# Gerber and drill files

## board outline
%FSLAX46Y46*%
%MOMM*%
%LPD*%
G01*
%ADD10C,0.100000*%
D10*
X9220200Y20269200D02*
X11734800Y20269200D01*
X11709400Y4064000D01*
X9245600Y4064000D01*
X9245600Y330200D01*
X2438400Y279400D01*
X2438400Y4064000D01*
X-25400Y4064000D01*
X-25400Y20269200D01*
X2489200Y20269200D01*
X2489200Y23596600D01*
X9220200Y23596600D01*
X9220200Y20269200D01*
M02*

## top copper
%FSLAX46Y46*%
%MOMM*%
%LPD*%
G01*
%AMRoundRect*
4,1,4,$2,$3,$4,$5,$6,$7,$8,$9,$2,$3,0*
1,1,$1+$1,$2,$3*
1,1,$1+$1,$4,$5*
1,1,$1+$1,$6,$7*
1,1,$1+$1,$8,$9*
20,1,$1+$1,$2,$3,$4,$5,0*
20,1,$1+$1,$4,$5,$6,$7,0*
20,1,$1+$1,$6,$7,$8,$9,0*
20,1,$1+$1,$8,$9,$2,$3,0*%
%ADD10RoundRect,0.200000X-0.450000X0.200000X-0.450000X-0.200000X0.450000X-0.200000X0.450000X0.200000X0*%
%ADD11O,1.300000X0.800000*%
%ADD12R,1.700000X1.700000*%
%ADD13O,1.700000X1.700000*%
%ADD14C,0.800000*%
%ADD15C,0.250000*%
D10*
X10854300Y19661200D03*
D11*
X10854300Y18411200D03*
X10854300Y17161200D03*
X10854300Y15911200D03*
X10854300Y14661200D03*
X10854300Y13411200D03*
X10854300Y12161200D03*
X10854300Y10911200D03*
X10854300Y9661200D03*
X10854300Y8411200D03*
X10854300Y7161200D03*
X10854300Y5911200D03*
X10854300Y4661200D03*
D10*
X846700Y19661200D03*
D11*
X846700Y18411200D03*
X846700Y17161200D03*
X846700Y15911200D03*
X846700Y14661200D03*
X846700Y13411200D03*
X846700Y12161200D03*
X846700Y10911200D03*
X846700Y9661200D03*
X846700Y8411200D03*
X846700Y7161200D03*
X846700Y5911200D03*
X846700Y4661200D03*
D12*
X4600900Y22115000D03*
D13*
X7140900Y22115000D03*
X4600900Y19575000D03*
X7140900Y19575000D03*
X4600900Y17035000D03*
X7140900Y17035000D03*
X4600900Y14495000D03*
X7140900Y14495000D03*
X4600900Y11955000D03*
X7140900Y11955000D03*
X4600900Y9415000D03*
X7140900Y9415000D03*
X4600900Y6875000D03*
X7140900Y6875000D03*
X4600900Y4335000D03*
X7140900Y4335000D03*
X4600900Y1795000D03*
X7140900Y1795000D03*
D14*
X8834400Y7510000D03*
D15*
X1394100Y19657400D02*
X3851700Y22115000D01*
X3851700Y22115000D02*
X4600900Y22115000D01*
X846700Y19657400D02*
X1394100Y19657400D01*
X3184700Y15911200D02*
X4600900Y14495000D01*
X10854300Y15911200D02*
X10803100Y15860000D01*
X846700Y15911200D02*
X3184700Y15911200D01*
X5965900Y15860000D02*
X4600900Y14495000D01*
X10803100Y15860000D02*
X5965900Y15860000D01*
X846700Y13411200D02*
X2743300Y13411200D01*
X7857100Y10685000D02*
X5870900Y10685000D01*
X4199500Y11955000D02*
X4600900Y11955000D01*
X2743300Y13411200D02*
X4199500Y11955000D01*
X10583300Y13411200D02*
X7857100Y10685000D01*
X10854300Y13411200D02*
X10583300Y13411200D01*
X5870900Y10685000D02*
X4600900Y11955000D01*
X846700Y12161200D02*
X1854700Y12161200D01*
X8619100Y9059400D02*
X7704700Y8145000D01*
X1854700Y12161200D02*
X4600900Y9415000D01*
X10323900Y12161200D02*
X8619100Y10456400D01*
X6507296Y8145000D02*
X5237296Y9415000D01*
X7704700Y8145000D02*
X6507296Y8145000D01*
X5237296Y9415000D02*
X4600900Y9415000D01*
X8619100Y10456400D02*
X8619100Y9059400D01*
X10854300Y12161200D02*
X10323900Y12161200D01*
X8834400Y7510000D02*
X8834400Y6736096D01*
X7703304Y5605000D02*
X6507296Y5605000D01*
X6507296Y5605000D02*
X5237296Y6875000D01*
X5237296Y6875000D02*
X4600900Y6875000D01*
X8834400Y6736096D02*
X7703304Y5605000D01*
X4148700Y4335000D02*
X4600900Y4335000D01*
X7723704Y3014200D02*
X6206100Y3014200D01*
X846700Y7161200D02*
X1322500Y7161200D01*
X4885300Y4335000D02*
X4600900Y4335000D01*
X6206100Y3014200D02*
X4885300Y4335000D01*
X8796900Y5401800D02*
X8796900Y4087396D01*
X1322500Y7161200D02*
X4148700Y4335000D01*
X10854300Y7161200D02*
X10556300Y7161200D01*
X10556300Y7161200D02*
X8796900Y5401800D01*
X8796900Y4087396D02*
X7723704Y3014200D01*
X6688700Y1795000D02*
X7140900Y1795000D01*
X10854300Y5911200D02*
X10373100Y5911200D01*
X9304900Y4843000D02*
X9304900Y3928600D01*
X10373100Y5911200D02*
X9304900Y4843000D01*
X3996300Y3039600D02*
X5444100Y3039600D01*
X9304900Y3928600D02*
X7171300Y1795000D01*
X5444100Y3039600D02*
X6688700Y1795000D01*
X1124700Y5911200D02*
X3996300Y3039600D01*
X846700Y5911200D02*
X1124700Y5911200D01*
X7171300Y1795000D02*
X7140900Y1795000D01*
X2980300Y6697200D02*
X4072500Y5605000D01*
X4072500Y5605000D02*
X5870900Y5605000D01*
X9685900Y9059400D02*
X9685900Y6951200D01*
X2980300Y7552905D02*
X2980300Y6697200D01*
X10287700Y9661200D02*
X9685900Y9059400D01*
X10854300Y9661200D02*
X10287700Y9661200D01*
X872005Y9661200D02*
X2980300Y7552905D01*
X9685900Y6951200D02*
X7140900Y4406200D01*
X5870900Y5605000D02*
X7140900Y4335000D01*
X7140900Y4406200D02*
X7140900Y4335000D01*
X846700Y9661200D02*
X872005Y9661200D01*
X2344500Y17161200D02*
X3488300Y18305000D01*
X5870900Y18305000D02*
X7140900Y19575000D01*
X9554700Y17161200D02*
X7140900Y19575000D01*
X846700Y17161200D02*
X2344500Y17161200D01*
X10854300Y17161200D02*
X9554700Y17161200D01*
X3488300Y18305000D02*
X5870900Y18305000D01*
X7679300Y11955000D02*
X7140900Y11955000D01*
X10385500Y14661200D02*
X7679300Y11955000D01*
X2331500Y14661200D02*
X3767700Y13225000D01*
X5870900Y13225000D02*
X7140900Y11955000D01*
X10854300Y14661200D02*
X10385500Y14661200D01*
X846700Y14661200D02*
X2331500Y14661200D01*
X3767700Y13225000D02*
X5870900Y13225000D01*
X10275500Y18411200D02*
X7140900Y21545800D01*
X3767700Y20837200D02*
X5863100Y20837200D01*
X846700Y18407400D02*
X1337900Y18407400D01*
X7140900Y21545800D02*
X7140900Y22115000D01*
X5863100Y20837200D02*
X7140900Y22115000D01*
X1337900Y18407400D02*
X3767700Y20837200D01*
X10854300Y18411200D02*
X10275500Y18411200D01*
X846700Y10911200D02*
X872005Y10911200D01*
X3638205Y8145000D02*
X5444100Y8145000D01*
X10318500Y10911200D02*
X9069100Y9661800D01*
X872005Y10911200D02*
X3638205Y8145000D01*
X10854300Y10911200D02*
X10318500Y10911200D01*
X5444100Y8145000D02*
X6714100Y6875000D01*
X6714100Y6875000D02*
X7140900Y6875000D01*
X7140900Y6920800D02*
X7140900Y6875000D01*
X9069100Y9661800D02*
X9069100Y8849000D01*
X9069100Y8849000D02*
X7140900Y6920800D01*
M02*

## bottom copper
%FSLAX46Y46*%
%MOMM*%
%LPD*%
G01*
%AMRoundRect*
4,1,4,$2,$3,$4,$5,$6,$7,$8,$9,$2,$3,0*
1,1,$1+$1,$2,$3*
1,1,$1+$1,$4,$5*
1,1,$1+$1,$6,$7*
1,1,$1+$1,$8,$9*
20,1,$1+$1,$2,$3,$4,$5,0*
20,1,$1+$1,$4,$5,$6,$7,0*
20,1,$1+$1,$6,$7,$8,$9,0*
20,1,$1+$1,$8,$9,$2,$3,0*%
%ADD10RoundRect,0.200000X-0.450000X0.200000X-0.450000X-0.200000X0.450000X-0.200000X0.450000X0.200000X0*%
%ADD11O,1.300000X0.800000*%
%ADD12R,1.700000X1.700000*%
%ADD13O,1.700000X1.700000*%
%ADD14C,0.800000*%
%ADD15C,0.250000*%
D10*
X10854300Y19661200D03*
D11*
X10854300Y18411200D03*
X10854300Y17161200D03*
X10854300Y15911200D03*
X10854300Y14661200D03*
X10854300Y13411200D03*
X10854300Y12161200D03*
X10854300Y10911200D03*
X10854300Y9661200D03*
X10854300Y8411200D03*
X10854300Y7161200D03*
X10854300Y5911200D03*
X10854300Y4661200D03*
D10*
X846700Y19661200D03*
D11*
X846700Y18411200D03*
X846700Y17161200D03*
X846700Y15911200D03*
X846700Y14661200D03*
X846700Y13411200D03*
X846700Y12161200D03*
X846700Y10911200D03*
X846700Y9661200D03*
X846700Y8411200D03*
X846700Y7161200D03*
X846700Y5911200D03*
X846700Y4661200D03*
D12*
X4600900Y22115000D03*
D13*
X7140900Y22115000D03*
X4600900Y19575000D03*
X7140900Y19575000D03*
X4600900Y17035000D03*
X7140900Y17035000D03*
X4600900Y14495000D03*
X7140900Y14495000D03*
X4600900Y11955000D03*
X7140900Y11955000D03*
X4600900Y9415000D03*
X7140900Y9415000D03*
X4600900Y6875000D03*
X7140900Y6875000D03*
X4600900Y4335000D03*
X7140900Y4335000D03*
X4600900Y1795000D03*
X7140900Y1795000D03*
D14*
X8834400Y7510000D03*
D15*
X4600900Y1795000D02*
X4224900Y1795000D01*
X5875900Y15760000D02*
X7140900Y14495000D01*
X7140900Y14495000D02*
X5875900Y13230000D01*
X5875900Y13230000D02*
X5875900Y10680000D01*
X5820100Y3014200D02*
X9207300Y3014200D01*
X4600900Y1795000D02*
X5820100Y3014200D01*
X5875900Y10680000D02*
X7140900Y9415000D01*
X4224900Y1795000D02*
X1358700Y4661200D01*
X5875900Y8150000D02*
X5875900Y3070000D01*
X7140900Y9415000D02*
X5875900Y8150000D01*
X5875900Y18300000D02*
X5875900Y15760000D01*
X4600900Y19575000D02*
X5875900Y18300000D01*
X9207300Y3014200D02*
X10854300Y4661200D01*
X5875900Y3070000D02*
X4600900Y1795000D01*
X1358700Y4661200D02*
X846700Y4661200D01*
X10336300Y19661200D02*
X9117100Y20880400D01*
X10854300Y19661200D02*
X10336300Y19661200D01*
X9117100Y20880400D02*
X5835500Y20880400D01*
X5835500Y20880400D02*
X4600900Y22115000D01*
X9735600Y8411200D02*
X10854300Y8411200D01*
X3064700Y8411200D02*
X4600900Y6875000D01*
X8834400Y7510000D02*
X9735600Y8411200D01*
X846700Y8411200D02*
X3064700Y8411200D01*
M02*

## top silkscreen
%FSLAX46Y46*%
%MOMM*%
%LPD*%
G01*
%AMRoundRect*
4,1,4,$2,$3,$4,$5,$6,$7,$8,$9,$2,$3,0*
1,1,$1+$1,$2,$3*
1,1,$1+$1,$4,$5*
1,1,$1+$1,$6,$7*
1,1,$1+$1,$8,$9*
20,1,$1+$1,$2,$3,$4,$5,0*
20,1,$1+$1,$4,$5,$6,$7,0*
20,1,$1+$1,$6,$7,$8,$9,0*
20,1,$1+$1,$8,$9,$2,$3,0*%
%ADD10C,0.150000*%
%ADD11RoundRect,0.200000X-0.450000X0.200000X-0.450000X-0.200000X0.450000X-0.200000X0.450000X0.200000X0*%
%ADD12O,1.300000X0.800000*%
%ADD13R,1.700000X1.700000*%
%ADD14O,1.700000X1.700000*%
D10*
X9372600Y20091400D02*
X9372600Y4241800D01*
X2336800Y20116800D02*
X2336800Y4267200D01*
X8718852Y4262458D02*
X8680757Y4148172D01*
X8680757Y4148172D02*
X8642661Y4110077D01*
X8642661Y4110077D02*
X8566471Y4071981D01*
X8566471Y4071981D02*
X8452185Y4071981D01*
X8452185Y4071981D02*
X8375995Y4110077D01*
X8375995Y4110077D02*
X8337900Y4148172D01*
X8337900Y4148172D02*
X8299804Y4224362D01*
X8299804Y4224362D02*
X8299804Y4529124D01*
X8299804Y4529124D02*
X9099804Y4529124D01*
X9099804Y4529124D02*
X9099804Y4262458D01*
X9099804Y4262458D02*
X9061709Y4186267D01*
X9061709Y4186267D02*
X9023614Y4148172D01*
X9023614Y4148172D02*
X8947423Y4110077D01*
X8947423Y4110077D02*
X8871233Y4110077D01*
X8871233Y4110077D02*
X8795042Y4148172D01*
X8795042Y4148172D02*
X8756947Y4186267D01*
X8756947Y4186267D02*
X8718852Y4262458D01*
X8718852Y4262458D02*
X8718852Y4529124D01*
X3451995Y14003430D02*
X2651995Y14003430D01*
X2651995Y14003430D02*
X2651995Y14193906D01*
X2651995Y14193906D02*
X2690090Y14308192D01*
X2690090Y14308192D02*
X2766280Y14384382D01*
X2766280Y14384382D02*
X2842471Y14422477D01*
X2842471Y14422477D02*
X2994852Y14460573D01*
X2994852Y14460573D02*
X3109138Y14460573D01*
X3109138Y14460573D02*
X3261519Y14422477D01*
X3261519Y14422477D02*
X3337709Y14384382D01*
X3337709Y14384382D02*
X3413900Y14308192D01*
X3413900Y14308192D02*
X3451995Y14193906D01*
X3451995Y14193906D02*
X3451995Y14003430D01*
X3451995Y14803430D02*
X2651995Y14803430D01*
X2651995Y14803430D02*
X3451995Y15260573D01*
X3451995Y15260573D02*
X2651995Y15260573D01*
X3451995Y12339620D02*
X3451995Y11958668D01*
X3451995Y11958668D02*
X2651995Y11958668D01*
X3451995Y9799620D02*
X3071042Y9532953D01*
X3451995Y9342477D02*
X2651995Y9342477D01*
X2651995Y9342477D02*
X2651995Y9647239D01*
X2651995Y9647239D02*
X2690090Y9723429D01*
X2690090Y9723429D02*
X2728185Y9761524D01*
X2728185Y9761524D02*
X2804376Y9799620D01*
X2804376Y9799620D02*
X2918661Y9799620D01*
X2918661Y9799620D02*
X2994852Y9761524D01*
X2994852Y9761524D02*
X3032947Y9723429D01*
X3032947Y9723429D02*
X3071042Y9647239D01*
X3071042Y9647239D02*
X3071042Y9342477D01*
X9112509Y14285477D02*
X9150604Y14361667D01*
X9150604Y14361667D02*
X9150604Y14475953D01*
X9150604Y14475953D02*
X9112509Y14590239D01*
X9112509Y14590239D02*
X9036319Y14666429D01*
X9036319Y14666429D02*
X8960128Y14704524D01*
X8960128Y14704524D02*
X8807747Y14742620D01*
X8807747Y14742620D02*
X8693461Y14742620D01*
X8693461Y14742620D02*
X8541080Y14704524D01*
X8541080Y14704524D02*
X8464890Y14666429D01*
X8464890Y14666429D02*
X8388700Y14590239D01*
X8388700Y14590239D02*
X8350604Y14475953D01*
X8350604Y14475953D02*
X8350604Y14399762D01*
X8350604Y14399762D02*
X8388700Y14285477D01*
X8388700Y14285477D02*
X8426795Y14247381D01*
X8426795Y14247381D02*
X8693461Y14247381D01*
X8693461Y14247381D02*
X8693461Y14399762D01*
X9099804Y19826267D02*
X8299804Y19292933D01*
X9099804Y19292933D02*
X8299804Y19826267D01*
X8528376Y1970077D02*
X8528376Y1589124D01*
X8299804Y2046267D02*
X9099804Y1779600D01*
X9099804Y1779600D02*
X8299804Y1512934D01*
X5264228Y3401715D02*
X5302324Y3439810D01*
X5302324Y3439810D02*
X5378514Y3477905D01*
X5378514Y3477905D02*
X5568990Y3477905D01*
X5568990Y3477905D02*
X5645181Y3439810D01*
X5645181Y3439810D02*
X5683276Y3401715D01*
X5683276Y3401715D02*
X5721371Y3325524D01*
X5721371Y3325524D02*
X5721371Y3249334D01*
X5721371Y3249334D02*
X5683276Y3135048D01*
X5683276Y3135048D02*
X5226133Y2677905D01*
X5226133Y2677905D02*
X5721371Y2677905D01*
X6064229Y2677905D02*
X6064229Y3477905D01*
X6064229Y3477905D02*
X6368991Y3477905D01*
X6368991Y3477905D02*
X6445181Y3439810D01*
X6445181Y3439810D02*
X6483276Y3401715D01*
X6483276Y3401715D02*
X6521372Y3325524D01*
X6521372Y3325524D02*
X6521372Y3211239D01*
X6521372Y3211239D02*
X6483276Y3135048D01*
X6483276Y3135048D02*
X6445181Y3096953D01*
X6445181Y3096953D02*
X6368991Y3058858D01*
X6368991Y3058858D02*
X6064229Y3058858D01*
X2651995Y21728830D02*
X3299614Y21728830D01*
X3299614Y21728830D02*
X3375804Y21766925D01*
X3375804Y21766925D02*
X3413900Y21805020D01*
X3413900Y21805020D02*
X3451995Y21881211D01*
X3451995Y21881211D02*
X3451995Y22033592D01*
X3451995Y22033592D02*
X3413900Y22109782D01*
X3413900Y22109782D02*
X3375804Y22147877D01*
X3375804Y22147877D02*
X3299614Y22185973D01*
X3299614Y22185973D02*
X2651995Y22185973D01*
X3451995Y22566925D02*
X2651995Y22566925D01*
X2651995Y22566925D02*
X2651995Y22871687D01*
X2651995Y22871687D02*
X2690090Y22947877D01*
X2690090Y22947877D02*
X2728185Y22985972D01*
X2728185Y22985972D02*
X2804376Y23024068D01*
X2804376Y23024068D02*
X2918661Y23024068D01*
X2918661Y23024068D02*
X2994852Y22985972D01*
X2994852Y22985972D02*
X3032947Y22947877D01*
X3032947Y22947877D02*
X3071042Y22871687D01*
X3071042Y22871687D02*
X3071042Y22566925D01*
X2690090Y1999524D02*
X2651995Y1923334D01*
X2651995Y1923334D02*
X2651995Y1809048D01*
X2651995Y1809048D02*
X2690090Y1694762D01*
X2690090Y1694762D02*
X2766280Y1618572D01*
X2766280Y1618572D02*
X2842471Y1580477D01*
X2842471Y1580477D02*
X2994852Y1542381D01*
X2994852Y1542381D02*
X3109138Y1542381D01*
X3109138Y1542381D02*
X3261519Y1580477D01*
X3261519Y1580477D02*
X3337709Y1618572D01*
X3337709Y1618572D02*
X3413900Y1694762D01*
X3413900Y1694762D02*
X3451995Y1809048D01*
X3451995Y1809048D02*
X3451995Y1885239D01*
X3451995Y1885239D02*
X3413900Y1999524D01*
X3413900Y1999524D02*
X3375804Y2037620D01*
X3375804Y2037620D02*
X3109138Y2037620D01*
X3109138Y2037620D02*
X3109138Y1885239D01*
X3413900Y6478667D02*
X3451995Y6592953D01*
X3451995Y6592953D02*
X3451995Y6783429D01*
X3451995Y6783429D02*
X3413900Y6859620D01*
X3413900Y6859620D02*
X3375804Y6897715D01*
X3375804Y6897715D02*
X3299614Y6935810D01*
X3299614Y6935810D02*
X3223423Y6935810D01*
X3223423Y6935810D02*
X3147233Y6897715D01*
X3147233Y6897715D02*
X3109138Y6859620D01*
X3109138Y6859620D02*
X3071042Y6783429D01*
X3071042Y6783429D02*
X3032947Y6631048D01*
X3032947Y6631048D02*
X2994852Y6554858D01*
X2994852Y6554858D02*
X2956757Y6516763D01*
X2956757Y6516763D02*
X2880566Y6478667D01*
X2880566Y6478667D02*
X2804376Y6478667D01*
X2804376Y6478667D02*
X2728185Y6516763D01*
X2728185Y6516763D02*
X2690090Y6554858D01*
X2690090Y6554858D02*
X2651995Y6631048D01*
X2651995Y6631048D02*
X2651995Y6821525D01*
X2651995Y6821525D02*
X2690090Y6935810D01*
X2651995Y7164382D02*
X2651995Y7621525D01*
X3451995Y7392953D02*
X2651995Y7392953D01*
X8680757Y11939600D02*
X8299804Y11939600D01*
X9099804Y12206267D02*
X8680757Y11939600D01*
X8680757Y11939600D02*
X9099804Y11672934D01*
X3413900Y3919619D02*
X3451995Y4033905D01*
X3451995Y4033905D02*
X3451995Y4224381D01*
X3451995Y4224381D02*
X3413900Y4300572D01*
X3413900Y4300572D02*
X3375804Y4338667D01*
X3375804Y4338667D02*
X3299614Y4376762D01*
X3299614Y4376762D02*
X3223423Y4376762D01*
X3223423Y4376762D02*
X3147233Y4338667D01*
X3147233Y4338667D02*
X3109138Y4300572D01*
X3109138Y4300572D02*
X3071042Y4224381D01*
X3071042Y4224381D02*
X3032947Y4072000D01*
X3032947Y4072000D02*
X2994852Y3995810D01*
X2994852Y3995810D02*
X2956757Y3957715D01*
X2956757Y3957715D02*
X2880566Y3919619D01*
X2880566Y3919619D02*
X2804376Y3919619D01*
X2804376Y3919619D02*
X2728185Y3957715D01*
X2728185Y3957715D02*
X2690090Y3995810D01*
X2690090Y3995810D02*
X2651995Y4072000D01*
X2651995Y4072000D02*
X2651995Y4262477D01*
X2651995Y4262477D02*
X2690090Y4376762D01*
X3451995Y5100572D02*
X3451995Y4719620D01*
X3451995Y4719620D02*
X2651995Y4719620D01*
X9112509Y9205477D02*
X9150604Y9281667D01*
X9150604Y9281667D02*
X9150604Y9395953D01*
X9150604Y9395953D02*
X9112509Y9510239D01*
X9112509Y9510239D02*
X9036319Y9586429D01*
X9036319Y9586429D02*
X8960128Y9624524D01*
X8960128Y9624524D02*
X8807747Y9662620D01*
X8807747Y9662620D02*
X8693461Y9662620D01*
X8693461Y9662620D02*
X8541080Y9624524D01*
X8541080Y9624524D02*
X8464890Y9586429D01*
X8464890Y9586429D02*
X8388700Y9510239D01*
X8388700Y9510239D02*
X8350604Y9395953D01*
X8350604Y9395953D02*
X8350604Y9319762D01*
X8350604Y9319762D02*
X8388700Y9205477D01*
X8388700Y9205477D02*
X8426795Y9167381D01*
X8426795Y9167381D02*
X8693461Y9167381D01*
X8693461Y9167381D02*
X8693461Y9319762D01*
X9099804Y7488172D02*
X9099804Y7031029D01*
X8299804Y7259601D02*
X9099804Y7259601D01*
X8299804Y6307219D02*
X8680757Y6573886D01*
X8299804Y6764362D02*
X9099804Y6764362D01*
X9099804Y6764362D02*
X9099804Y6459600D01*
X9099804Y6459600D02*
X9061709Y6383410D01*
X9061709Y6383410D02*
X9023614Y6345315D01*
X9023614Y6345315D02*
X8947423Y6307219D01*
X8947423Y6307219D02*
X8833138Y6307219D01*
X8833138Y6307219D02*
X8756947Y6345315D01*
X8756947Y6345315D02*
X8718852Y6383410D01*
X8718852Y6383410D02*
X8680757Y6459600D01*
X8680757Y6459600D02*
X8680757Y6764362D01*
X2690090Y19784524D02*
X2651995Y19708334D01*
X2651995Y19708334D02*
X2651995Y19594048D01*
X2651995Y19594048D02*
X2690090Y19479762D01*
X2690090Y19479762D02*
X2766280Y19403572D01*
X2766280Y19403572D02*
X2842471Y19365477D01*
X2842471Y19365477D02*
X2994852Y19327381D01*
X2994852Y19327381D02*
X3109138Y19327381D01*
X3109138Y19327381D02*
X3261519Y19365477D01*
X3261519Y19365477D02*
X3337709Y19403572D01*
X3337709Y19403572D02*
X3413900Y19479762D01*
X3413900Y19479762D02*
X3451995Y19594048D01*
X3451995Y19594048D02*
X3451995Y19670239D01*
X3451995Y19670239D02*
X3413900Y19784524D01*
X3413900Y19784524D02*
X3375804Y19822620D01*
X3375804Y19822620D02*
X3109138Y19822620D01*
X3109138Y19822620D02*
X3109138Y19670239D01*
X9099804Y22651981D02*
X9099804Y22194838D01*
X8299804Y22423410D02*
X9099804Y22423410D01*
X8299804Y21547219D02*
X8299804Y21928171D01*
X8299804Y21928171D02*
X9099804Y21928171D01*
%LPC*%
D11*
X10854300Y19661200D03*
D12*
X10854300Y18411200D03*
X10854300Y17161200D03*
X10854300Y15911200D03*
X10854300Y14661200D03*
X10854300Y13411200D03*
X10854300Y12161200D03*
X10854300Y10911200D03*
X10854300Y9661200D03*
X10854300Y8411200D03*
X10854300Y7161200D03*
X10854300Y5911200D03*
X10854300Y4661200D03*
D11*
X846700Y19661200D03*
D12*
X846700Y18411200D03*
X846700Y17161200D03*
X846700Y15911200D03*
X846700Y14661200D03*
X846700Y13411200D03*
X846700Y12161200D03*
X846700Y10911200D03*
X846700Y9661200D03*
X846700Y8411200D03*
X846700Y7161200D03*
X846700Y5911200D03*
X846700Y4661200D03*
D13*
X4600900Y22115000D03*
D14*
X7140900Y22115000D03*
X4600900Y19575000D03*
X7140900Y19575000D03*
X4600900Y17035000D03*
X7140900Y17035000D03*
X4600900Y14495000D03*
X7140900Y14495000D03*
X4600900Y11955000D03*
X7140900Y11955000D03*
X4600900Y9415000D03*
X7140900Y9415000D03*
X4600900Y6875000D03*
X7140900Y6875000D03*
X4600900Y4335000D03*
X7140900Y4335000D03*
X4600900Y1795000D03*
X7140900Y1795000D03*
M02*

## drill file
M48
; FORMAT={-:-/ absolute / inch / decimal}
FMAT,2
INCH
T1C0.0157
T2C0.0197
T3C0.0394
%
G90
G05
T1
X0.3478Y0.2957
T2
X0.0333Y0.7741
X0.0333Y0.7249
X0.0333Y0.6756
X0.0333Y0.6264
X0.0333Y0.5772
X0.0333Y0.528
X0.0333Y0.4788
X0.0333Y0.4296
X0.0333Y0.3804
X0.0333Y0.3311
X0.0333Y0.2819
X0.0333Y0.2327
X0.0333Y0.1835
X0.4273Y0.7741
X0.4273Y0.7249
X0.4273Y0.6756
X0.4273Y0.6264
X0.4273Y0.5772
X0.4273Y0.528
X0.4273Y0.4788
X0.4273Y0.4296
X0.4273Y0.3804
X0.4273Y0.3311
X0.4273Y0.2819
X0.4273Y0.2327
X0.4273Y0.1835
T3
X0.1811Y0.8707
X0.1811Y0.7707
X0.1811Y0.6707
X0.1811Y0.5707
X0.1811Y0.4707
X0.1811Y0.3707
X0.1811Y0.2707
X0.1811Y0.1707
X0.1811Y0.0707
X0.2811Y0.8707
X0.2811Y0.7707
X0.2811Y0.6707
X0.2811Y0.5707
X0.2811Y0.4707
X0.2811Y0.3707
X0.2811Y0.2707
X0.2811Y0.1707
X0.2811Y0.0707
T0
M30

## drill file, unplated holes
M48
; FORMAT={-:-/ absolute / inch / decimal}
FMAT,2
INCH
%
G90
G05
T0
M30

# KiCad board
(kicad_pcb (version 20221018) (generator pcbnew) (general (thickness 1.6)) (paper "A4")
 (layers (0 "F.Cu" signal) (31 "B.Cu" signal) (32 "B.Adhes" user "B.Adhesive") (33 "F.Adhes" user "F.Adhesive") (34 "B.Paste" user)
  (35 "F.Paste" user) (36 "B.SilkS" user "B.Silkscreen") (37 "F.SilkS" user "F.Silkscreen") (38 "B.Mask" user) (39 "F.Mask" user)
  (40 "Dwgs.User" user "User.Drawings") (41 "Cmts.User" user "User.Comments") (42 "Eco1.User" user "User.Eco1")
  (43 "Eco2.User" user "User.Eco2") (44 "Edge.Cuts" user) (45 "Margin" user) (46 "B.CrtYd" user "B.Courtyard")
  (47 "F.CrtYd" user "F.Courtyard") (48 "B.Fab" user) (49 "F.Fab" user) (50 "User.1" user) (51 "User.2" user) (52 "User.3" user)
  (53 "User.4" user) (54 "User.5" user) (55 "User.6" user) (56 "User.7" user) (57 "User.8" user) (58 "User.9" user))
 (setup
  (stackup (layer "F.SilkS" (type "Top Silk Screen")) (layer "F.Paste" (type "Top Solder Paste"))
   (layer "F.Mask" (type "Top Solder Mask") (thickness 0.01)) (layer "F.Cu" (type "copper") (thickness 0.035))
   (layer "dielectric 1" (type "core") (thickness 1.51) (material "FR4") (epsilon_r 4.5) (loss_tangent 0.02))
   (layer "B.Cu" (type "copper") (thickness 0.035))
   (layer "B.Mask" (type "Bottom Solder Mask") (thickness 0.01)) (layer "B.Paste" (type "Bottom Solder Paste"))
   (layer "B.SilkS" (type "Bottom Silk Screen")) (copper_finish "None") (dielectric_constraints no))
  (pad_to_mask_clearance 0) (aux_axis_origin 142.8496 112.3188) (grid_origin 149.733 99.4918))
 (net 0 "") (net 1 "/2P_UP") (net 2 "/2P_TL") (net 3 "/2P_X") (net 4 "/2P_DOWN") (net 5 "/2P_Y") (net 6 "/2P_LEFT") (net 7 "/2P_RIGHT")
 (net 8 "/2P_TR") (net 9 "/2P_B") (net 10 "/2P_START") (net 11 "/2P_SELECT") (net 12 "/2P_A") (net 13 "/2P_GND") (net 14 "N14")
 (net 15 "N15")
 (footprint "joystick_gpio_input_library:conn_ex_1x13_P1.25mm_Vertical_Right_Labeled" (layer "B.Cu") (at 153.7039 92.6576 -90)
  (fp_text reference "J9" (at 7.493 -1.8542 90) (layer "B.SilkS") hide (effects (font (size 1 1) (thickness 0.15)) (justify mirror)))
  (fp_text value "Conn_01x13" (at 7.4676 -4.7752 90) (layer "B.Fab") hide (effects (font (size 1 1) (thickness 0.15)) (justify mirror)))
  (pad "1" thru_hole roundrect (at 0 0 270) (size 0.8 1.3) (drill 0.5) (layers "*.Cu" "*.Mask") (roundrect_rratio 0.25) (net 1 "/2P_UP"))
  (pad "2" thru_hole oval (at 1.25 0 270) (size 0.8 1.3) (drill 0.5) (layers "*.Cu" "*.Mask") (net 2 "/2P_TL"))
  (pad "3" thru_hole oval (at 2.5 0 270) (size 0.8 1.3) (drill 0.5) (layers "*.Cu" "*.Mask") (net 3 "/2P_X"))
  (pad "4" thru_hole oval (at 3.75 0 270) (size 0.8 1.3) (drill 0.5) (layers "*.Cu" "*.Mask") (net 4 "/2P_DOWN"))
  (pad "5" thru_hole oval (at 5 0 270) (size 0.8 1.3) (drill 0.5) (layers "*.Cu" "*.Mask") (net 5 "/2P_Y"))
  (pad "6" thru_hole oval (at 6.25 0 270) (size 0.8 1.3) (drill 0.5) (layers "*.Cu" "*.Mask") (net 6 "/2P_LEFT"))
  (pad "7" thru_hole oval (at 7.5 0 270) (size 0.8 1.3) (drill 0.5) (layers "*.Cu" "*.Mask") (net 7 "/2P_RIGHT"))
  (pad "8" thru_hole oval (at 8.75 0 270) (size 0.8 1.3) (drill 0.5) (layers "*.Cu" "*.Mask") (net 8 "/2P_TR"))
  (pad "9" thru_hole oval (at 10 0 270) (size 0.8 1.3) (drill 0.5) (layers "*.Cu" "*.Mask") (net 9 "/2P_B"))
  (pad "10" thru_hole oval (at 11.25 0 270) (size 0.8 1.3) (drill 0.5) (layers "*.Cu" "*.Mask") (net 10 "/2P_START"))
  (pad "11" thru_hole oval (at 12.5 0 270) (size 0.8 1.3) (drill 0.5) (layers "*.Cu" "*.Mask") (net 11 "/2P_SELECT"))
  (pad "12" thru_hole oval (at 13.75 0 270) (size 0.8 1.3) (drill 0.5) (layers "*.Cu" "*.Mask") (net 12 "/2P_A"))
  (pad "13" thru_hole oval (at 15 0 270) (size 0.8 1.3) (drill 0.5) (layers "*.Cu" "*.Mask") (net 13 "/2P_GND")))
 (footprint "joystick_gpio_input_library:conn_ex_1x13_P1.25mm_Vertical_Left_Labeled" (layer "B.Cu") (at 143.6963 92.6576 -90)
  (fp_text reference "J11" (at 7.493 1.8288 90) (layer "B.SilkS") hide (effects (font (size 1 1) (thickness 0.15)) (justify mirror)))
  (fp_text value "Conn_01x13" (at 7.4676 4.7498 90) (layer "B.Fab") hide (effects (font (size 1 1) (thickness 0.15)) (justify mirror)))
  (pad "1" thru_hole roundrect (at 0 0 270) (size 0.8 1.3) (drill 0.5) (layers "*.Cu" "*.Mask") (roundrect_rratio 0.25) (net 1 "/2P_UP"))
  (pad "2" thru_hole oval (at 1.25 0 270) (size 0.8 1.3) (drill 0.5) (layers "*.Cu" "*.Mask") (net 2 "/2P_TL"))
  (pad "3" thru_hole oval (at 2.5 0 270) (size 0.8 1.3) (drill 0.5) (layers "*.Cu" "*.Mask") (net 3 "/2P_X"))
  (pad "4" thru_hole oval (at 3.75 0 270) (size 0.8 1.3) (drill 0.5) (layers "*.Cu" "*.Mask") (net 4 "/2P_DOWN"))
  (pad "5" thru_hole oval (at 5 0 270) (size 0.8 1.3) (drill 0.5) (layers "*.Cu" "*.Mask") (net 5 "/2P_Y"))
  (pad "6" thru_hole oval (at 6.25 0 270) (size 0.8 1.3) (drill 0.5) (layers "*.Cu" "*.Mask") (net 6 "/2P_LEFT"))
  (pad "7" thru_hole oval (at 7.5 0 270) (size 0.8 1.3) (drill 0.5) (layers "*.Cu" "*.Mask") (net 7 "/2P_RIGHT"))
  (pad "8" thru_hole oval (at 8.75 0 270) (size 0.8 1.3) (drill 0.5) (layers "*.Cu" "*.Mask") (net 8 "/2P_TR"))
  (pad "9" thru_hole oval (at 10 0 270) (size 0.8 1.3) (drill 0.5) (layers "*.Cu" "*.Mask") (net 9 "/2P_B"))
  (pad "10" thru_hole oval (at 11.25 0 270) (size 0.8 1.3) (drill 0.5) (layers "*.Cu" "*.Mask") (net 10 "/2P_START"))
  (pad "11" thru_hole oval (at 12.5 0 270) (size 0.8 1.3) (drill 0.5) (layers "*.Cu" "*.Mask") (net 11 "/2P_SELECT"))
  (pad "12" thru_hole oval (at 13.75 0 270) (size 0.8 1.3) (drill 0.5) (layers "*.Cu" "*.Mask") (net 12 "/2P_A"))
  (pad "13" thru_hole oval (at 15 0 270) (size 0.8 1.3) (drill 0.5) (layers "*.Cu" "*.Mask") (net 13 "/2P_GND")))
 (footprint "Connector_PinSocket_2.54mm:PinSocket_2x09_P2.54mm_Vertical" (layer "B.Cu") (at 147.4505 90.2038 180)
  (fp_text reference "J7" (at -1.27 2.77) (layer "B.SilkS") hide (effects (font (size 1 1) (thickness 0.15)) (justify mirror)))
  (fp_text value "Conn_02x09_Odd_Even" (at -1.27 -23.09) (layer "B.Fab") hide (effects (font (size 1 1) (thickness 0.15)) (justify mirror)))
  (pad "1" thru_hole rect (at 0 0 180) (size 1.7 1.7) (drill 1) (layers "*.Cu" "*.Mask") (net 1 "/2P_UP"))
  (pad "2" thru_hole oval (at -2.54 0 180) (size 1.7 1.7) (drill 1) (layers "*.Cu" "*.Mask") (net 2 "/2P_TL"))
  (pad "3" thru_hole oval (at 0 -2.54 180) (size 1.7 1.7) (drill 1) (layers "*.Cu" "*.Mask") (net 13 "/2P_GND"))
  (pad "4" thru_hole oval (at -2.54 -2.54 180) (size 1.7 1.7) (drill 1) (layers "*.Cu" "*.Mask") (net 3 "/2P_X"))
  (pad "5" thru_hole oval (at 0 -5.08 180) (size 1.7 1.7) (drill 1) (layers "*.Cu" "*.Mask") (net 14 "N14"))
  (pad "6" thru_hole oval (at -2.54 -5.08 180) (size 1.7 1.7) (drill 1) (layers "*.Cu" "*.Mask") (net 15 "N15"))
  (pad "7" thru_hole oval (at 0 -7.62 180) (size 1.7 1.7) (drill 1) (layers "*.Cu" "*.Mask") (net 4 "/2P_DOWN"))
  (pad "8" thru_hole oval (at -2.54 -7.62 180) (size 1.7 1.7) (drill 1) (layers "*.Cu" "*.Mask") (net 13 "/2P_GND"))
  (pad "9" thru_hole oval (at 0 -10.16 180) (size 1.7 1.7) (drill 1) (layers "*.Cu" "*.Mask") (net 6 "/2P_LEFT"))
  (pad "10" thru_hole oval (at -2.54 -10.16 180) (size 1.7 1.7) (drill 1) (layers "*.Cu" "*.Mask") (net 5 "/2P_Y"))
  (pad "11" thru_hole oval (at 0 -12.7 180) (size 1.7 1.7) (drill 1) (layers "*.Cu" "*.Mask") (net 7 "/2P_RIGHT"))
  (pad "12" thru_hole oval (at -2.54 -12.7 180) (size 1.7 1.7) (drill 1) (layers "*.Cu" "*.Mask") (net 13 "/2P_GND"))
  (pad "13" thru_hole oval (at 0 -15.24 180) (size 1.7 1.7) (drill 1) (layers "*.Cu" "*.Mask") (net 10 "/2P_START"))
  (pad "14" thru_hole oval (at -2.54 -15.24 180) (size 1.7 1.7) (drill 1) (layers "*.Cu" "*.Mask") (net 8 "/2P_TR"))
  (pad "15" thru_hole oval (at 0 -17.78 180) (size 1.7 1.7) (drill 1) (layers "*.Cu" "*.Mask") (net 11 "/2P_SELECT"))
  (pad "16" thru_hole oval (at -2.54 -17.78 180) (size 1.7 1.7) (drill 1) (layers "*.Cu" "*.Mask") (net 9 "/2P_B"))
  (pad "17" thru_hole oval (at 0 -20.32 180) (size 1.7 1.7) (drill 1) (layers "*.Cu" "*.Mask") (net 13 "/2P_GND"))
  (pad "18" thru_hole oval (at -2.54 -20.32 180) (size 1.7 1.7) (drill 1) (layers "*.Cu" "*.Mask") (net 12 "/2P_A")))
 (gr_line (start 152.2222 92.2274) (end 152.2222 108.077) (stroke (width 0.15) (type default)) (layer "F.SilkS"))
 (gr_line (start 145.1864 92.202) (end 145.1864 108.0516) (stroke (width 0.15) (type default)) (layer "F.SilkS"))
 (gr_poly
  (pts (xy 145.3388 92.0496) (xy 145.3388 88.7222) (xy 152.0698 88.7222) (xy 152.0698 92.0496) (xy 154.5844 92.0496) (xy 154.559 108.2548)
   (xy 152.0952 108.2548) (xy 152.0952 111.9886) (xy 145.288 112.0394) (xy 145.288 108.2548) (xy 142.8242 108.2548) (xy 142.8242 92.0496))
  (stroke (width 0.1) (type solid)) (fill none) (layer "Edge.Cuts"))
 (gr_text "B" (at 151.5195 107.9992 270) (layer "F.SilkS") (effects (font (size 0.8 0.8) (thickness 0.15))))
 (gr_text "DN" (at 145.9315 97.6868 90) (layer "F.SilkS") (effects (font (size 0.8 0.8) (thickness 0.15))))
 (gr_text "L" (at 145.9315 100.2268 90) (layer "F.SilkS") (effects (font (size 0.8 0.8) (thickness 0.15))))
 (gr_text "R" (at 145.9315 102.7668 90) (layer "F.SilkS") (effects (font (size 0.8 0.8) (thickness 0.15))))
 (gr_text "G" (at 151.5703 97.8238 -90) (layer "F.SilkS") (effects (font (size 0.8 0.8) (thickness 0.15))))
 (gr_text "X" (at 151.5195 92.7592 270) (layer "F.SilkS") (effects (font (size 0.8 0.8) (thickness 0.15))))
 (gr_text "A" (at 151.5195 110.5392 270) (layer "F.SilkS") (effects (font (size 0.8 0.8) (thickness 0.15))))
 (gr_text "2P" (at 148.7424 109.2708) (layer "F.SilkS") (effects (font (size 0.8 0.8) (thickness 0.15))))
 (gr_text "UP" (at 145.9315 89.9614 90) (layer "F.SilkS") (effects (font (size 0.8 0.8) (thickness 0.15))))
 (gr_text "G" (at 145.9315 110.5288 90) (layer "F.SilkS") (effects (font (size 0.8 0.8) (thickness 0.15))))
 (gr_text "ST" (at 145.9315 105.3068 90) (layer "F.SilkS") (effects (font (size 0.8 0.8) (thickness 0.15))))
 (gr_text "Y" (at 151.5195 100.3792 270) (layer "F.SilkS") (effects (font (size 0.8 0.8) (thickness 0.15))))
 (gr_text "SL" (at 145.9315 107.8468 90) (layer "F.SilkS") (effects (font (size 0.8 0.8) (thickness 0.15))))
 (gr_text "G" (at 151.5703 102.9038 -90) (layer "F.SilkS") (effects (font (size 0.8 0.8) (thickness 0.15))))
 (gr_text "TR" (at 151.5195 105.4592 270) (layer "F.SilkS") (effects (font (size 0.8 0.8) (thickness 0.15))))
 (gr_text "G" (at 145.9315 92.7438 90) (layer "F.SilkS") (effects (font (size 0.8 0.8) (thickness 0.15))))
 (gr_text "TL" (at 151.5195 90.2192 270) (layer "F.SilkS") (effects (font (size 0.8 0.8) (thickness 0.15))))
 (segment (start 147.4505 110.5238) (end 147.0745 110.5238) (width 0.25) (layer "B.Cu") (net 13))
 (segment (start 148.7255 96.5588) (end 149.9905 97.8238) (width 0.25) (layer "B.Cu") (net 13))
 (segment (start 149.9905 97.8238) (end 148.7255 99.0888) (width 0.25) (layer "B.Cu") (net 13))
 (segment (start 148.7255 99.0888) (end 148.7255 101.6388) (width 0.25) (layer "B.Cu") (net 13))
 (segment (start 148.6697 109.3046) (end 152.0569 109.3046) (width 0.25) (layer "B.Cu") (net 13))
 (segment (start 147.4505 110.5238) (end 148.6697 109.3046) (width 0.25) (layer "B.Cu") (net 13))
 (segment (start 148.7255 101.6388) (end 149.9905 102.9038) (width 0.25) (layer "B.Cu") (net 13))
 (segment (start 147.0745 110.5238) (end 144.2083 107.6576) (width 0.25) (layer "B.Cu") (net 13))
 (segment (start 148.7255 104.1688) (end 148.7255 109.2488) (width 0.25) (layer "B.Cu") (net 13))
 (segment (start 149.9905 102.9038) (end 148.7255 104.1688) (width 0.25) (layer "B.Cu") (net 13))
 (segment (start 148.7255 94.0188) (end 148.7255 96.5588) (width 0.25) (layer "B.Cu") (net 13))
 (segment (start 147.4505 92.7438) (end 148.7255 94.0188) (width 0.25) (layer "B.Cu") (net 13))
 (segment (start 152.0569 109.3046) (end 153.7039 107.6576) (width 0.25) (layer "B.Cu") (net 13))
 (segment (start 148.7255 109.2488) (end 147.4505 110.5238) (width 0.25) (layer "B.Cu") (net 13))
 (segment (start 144.2083 107.6576) (end 143.6963 107.6576) (width 0.25) (layer "B.Cu") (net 13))
 (segment (start 144.2437 92.6614) (end 146.7013 90.2038) (width 0.25) (layer "F.Cu") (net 1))
 (segment (start 146.7013 90.2038) (end 147.4505 90.2038) (width 0.25) (layer "F.Cu") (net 1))
 (segment (start 143.6963 92.6614) (end 144.2437 92.6614) (width 0.25) (layer "F.Cu") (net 1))
 (segment (start 153.1859 92.6576) (end 151.9667 91.4384) (width 0.25) (layer "B.Cu") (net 1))
 (segment (start 153.7039 92.6576) (end 153.1859 92.6576) (width 0.25) (layer "B.Cu") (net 1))
 (segment (start 151.9667 91.4384) (end 148.6851 91.4384) (width 0.25) (layer "B.Cu") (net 1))
 (segment (start 148.6851 91.4384) (end 147.4505 90.2038) (width 0.25) (layer "B.Cu") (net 1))
 (segment (start 146.0343 96.4076) (end 147.4505 97.8238) (width 0.25) (layer "F.Cu") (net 4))
 (segment (start 153.7039 96.4076) (end 153.6527 96.4588) (width 0.25) (layer "F.Cu") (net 4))
 (segment (start 143.6963 96.4076) (end 146.0343 96.4076) (width 0.25) (layer "F.Cu") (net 4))
 (segment (start 148.8155 96.4588) (end 147.4505 97.8238) (width 0.25) (layer "F.Cu") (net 4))
 (segment (start 153.6527 96.4588) (end 148.8155 96.4588) (width 0.25) (layer "F.Cu") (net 4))
 (segment (start 143.6963 98.9076) (end 145.5929 98.9076) (width 0.25) (layer "F.Cu") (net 6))
 (segment (start 150.7067 101.6338) (end 148.7205 101.6338) (width 0.25) (layer "F.Cu") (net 6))
 (segment (start 147.0491 100.3638) (end 147.4505 100.3638) (width 0.25) (layer "F.Cu") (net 6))
 (segment (start 145.5929 98.9076) (end 147.0491 100.3638) (width 0.25) (layer "F.Cu") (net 6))
 (segment (start 153.4329 98.9076) (end 150.7067 101.6338) (width 0.25) (layer "F.Cu") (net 6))
 (segment (start 153.7039 98.9076) (end 153.4329 98.9076) (width 0.25) (layer "F.Cu") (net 6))
 (segment (start 148.7205 101.6338) (end 147.4505 100.3638) (width 0.25) (layer "F.Cu") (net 6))
 (segment (start 143.6963 100.1576) (end 144.7043 100.1576) (width 0.25) (layer "F.Cu") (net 7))
 (segment (start 151.4687 103.2594) (end 150.5543 104.1738) (width 0.25) (layer "F.Cu") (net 7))
 (segment (start 144.7043 100.1576) (end 147.4505 102.9038) (width 0.25) (layer "F.Cu") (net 7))
 (segment (start 153.1735 100.1576) (end 151.4687 101.8624) (width 0.25) (layer "F.Cu") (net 7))
 (segment (start 149.356896 104.1738) (end 148.086896 102.9038) (width 0.25) (layer "F.Cu") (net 7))
 (segment (start 150.5543 104.1738) (end 149.356896 104.1738) (width 0.25) (layer "F.Cu") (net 7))
 (segment (start 148.086896 102.9038) (end 147.4505 102.9038) (width 0.25) (layer "F.Cu") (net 7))
 (segment (start 151.4687 101.8624) (end 151.4687 103.2594) (width 0.25) (layer "F.Cu") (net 7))
 (segment (start 153.7039 100.1576) (end 153.1735 100.1576) (width 0.25) (layer "F.Cu") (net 7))
 (segment (start 151.684 104.8088) (end 151.684 105.582704) (width 0.25) (layer "F.Cu") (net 10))
 (segment (start 150.552904 106.7138) (end 149.356896 106.7138) (width 0.25) (layer "F.Cu") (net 10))
 (segment (start 149.356896 106.7138) (end 148.086896 105.4438) (width 0.25) (layer "F.Cu") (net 10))
 (segment (start 148.086896 105.4438) (end 147.4505 105.4438) (width 0.25) (layer "F.Cu") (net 10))
 (segment (start 151.684 105.582704) (end 150.552904 106.7138) (width 0.25) (layer "F.Cu") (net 10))
 (via (at 151.684 104.8088) (size 0.8) (drill 0.4) (layers "F.Cu" "B.Cu") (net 10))
 (segment (start 152.5852 103.9076) (end 153.7039 103.9076) (width 0.25) (layer "B.Cu") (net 10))
 (segment (start 145.9143 103.9076) (end 147.4505 105.4438) (width 0.25) (layer "B.Cu") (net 10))
 (segment (start 151.684 104.8088) (end 152.5852 103.9076) (width 0.25) (layer "B.Cu") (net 10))
 (segment (start 143.6963 103.9076) (end 145.9143 103.9076) (width 0.25) (layer "B.Cu") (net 10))
 (segment (start 146.9983 107.9838) (end 147.4505 107.9838) (width 0.25) (layer "F.Cu") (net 11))
 (segment (start 150.573304 109.3046) (end 149.0557 109.3046) (width 0.25) (layer "F.Cu") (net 11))
 (segment (start 143.6963 105.1576) (end 144.1721 105.1576) (width 0.25) (layer "F.Cu") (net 11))
 (segment (start 147.7349 107.9838) (end 147.4505 107.9838) (width 0.25) (layer "F.Cu") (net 11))
 (segment (start 149.0557 109.3046) (end 147.7349 107.9838) (width 0.25) (layer "F.Cu") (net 11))
 (segment (start 151.6465 106.917) (end 151.6465 108.231404) (width 0.25) (layer "F.Cu") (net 11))
 (segment (start 144.1721 105.1576) (end 146.9983 107.9838) (width 0.25) (layer "F.Cu") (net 11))
 (segment (start 153.7039 105.1576) (end 153.4059 105.1576) (width 0.25) (layer "F.Cu") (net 11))
 (segment (start 153.4059 105.1576) (end 151.6465 106.917) (width 0.25) (layer "F.Cu") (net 11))
 (segment (start 151.6465 108.231404) (end 150.573304 109.3046) (width 0.25) (layer "F.Cu") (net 11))
 (segment (start 149.5383 110.5238) (end 149.9905 110.5238) (width 0.25) (layer "F.Cu") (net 12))
 (segment (start 153.7039 106.4076) (end 153.2227 106.4076) (width 0.25) (layer "F.Cu") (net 12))
 (segment (start 152.1545 107.4758) (end 152.1545 108.3902) (width 0.25) (layer "F.Cu") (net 12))
 (segment (start 153.2227 106.4076) (end 152.1545 107.4758) (width 0.25) (layer "F.Cu") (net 12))
 (segment (start 146.8459 109.2792) (end 148.2937 109.2792) (width 0.25) (layer "F.Cu") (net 12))
 (segment (start 152.1545 108.3902) (end 150.0209 110.5238) (width 0.25) (layer "F.Cu") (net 12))
 (segment (start 148.2937 109.2792) (end 149.5383 110.5238) (width 0.25) (layer "F.Cu") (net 12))
 (segment (start 143.9743 106.4076) (end 146.8459 109.2792) (width 0.25) (layer "F.Cu") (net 12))
 (segment (start 143.6963 106.4076) (end 143.9743 106.4076) (width 0.25) (layer "F.Cu") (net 12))
 (segment (start 150.0209 110.5238) (end 149.9905 110.5238) (width 0.25) (layer "F.Cu") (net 12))
 (segment (start 145.8299 105.6216) (end 146.9221 106.7138) (width 0.25) (layer "F.Cu") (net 9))
 (segment (start 146.9221 106.7138) (end 148.7205 106.7138) (width 0.25) (layer "F.Cu") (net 9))
 (segment (start 152.5355 103.2594) (end 152.5355 105.3676) (width 0.25) (layer "F.Cu") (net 9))
 (segment (start 145.8299 104.765895) (end 145.8299 105.6216) (width 0.25) (layer "F.Cu") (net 9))
 (segment (start 153.1373 102.6576) (end 152.5355 103.2594) (width 0.25) (layer "F.Cu") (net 9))
 (segment (start 153.7039 102.6576) (end 153.1373 102.6576) (width 0.25) (layer "F.Cu") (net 9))
 (segment (start 143.721605 102.6576) (end 145.8299 104.765895) (width 0.25) (layer "F.Cu") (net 9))
 (segment (start 152.5355 105.3676) (end 149.9905 107.9126) (width 0.25) (layer "F.Cu") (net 9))
 (segment (start 148.7205 106.7138) (end 149.9905 107.9838) (width 0.25) (layer "F.Cu") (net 9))
 (segment (start 149.9905 107.9126) (end 149.9905 107.9838) (width 0.25) (layer "F.Cu") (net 9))
 (segment (start 143.6963 102.6576) (end 143.721605 102.6576) (width 0.25) (layer "F.Cu") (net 9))
 (segment (start 145.1941 95.1576) (end 146.3379 94.0138) (width 0.25) (layer "F.Cu") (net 3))
 (segment (start 148.7205 94.0138) (end 149.9905 92.7438) (width 0.25) (layer "F.Cu") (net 3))
 (segment (start 152.4043 95.1576) (end 149.9905 92.7438) (width 0.25) (layer "F.Cu") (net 3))
 (segment (start 143.6963 95.1576) (end 145.1941 95.1576) (width 0.25) (layer "F.Cu") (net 3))
 (segment (start 153.7039 95.1576) (end 152.4043 95.1576) (width 0.25) (layer "F.Cu") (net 3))
 (segment (start 146.3379 94.0138) (end 148.7205 94.0138) (width 0.25) (layer "F.Cu") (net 3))
 (segment (start 150.5289 100.3638) (end 149.9905 100.3638) (width 0.25) (layer "F.Cu") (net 5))
 (segment (start 153.2351 97.6576) (end 150.5289 100.3638) (width 0.25) (layer "F.Cu") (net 5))
 (segment (start 145.1811 97.6576) (end 146.6173 99.0938) (width 0.25) (layer "F.Cu") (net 5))
 (segment (start 148.7205 99.0938) (end 149.9905 100.3638) (width 0.25) (layer "F.Cu") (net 5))
 (segment (start 153.7039 97.6576) (end 153.2351 97.6576) (width 0.25) (layer "F.Cu") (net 5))
 (segment (start 143.6963 97.6576) (end 145.1811 97.6576) (width 0.25) (layer "F.Cu") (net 5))
 (segment (start 146.6173 99.0938) (end 148.7205 99.0938) (width 0.25) (layer "F.Cu") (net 5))
 (segment (start 153.1251 93.9076) (end 149.9905 90.773) (width 0.25) (layer "F.Cu") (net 2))
 (segment (start 146.6173 91.4816) (end 148.7127 91.4816) (width 0.25) (layer "F.Cu") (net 2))
 (segment (start 143.6963 93.9114) (end 144.1875 93.9114) (width 0.25) (layer "F.Cu") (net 2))
 (segment (start 149.9905 90.773) (end 149.9905 90.2038) (width 0.25) (layer "F.Cu") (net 2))
 (segment (start 148.7127 91.4816) (end 149.9905 90.2038) (width 0.25) (layer "F.Cu") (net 2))
 (segment (start 144.1875 93.9114) (end 146.6173 91.4816) (width 0.25) (layer "F.Cu") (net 2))
 (segment (start 153.7039 93.9076) (end 153.1251 93.9076) (width 0.25) (layer "F.Cu") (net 2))
 (segment (start 143.6963 101.4076) (end 143.721605 101.4076) (width 0.25) (layer "F.Cu") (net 8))
 (segment (start 146.487805 104.1738) (end 148.2937 104.1738) (width 0.25) (layer "F.Cu") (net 8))
 (segment (start 153.1681 101.4076) (end 151.9187 102.657) (width 0.25) (layer "F.Cu") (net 8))
 (segment (start 143.721605 101.4076) (end 146.487805 104.1738) (width 0.25) (layer "F.Cu") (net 8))
 (segment (start 153.7039 101.4076) (end 153.1681 101.4076) (width 0.25) (layer "F.Cu") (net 8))
 (segment (start 148.2937 104.1738) (end 149.5637 105.4438) (width 0.25) (layer "F.Cu") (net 8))
 (segment (start 149.5637 105.4438) (end 149.9905 105.4438) (width 0.25) (layer "F.Cu") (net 8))
 (segment (start 149.9905 105.398) (end 149.9905 105.4438) (width 0.25) (layer "F.Cu") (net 8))
 (segment (start 151.9187 102.657) (end 151.9187 103.4698) (width 0.25) (layer "F.Cu") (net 8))
 (segment (start 151.9187 103.4698) (end 149.9905 105.398) (width 0.25) (layer "F.Cu") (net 8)))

